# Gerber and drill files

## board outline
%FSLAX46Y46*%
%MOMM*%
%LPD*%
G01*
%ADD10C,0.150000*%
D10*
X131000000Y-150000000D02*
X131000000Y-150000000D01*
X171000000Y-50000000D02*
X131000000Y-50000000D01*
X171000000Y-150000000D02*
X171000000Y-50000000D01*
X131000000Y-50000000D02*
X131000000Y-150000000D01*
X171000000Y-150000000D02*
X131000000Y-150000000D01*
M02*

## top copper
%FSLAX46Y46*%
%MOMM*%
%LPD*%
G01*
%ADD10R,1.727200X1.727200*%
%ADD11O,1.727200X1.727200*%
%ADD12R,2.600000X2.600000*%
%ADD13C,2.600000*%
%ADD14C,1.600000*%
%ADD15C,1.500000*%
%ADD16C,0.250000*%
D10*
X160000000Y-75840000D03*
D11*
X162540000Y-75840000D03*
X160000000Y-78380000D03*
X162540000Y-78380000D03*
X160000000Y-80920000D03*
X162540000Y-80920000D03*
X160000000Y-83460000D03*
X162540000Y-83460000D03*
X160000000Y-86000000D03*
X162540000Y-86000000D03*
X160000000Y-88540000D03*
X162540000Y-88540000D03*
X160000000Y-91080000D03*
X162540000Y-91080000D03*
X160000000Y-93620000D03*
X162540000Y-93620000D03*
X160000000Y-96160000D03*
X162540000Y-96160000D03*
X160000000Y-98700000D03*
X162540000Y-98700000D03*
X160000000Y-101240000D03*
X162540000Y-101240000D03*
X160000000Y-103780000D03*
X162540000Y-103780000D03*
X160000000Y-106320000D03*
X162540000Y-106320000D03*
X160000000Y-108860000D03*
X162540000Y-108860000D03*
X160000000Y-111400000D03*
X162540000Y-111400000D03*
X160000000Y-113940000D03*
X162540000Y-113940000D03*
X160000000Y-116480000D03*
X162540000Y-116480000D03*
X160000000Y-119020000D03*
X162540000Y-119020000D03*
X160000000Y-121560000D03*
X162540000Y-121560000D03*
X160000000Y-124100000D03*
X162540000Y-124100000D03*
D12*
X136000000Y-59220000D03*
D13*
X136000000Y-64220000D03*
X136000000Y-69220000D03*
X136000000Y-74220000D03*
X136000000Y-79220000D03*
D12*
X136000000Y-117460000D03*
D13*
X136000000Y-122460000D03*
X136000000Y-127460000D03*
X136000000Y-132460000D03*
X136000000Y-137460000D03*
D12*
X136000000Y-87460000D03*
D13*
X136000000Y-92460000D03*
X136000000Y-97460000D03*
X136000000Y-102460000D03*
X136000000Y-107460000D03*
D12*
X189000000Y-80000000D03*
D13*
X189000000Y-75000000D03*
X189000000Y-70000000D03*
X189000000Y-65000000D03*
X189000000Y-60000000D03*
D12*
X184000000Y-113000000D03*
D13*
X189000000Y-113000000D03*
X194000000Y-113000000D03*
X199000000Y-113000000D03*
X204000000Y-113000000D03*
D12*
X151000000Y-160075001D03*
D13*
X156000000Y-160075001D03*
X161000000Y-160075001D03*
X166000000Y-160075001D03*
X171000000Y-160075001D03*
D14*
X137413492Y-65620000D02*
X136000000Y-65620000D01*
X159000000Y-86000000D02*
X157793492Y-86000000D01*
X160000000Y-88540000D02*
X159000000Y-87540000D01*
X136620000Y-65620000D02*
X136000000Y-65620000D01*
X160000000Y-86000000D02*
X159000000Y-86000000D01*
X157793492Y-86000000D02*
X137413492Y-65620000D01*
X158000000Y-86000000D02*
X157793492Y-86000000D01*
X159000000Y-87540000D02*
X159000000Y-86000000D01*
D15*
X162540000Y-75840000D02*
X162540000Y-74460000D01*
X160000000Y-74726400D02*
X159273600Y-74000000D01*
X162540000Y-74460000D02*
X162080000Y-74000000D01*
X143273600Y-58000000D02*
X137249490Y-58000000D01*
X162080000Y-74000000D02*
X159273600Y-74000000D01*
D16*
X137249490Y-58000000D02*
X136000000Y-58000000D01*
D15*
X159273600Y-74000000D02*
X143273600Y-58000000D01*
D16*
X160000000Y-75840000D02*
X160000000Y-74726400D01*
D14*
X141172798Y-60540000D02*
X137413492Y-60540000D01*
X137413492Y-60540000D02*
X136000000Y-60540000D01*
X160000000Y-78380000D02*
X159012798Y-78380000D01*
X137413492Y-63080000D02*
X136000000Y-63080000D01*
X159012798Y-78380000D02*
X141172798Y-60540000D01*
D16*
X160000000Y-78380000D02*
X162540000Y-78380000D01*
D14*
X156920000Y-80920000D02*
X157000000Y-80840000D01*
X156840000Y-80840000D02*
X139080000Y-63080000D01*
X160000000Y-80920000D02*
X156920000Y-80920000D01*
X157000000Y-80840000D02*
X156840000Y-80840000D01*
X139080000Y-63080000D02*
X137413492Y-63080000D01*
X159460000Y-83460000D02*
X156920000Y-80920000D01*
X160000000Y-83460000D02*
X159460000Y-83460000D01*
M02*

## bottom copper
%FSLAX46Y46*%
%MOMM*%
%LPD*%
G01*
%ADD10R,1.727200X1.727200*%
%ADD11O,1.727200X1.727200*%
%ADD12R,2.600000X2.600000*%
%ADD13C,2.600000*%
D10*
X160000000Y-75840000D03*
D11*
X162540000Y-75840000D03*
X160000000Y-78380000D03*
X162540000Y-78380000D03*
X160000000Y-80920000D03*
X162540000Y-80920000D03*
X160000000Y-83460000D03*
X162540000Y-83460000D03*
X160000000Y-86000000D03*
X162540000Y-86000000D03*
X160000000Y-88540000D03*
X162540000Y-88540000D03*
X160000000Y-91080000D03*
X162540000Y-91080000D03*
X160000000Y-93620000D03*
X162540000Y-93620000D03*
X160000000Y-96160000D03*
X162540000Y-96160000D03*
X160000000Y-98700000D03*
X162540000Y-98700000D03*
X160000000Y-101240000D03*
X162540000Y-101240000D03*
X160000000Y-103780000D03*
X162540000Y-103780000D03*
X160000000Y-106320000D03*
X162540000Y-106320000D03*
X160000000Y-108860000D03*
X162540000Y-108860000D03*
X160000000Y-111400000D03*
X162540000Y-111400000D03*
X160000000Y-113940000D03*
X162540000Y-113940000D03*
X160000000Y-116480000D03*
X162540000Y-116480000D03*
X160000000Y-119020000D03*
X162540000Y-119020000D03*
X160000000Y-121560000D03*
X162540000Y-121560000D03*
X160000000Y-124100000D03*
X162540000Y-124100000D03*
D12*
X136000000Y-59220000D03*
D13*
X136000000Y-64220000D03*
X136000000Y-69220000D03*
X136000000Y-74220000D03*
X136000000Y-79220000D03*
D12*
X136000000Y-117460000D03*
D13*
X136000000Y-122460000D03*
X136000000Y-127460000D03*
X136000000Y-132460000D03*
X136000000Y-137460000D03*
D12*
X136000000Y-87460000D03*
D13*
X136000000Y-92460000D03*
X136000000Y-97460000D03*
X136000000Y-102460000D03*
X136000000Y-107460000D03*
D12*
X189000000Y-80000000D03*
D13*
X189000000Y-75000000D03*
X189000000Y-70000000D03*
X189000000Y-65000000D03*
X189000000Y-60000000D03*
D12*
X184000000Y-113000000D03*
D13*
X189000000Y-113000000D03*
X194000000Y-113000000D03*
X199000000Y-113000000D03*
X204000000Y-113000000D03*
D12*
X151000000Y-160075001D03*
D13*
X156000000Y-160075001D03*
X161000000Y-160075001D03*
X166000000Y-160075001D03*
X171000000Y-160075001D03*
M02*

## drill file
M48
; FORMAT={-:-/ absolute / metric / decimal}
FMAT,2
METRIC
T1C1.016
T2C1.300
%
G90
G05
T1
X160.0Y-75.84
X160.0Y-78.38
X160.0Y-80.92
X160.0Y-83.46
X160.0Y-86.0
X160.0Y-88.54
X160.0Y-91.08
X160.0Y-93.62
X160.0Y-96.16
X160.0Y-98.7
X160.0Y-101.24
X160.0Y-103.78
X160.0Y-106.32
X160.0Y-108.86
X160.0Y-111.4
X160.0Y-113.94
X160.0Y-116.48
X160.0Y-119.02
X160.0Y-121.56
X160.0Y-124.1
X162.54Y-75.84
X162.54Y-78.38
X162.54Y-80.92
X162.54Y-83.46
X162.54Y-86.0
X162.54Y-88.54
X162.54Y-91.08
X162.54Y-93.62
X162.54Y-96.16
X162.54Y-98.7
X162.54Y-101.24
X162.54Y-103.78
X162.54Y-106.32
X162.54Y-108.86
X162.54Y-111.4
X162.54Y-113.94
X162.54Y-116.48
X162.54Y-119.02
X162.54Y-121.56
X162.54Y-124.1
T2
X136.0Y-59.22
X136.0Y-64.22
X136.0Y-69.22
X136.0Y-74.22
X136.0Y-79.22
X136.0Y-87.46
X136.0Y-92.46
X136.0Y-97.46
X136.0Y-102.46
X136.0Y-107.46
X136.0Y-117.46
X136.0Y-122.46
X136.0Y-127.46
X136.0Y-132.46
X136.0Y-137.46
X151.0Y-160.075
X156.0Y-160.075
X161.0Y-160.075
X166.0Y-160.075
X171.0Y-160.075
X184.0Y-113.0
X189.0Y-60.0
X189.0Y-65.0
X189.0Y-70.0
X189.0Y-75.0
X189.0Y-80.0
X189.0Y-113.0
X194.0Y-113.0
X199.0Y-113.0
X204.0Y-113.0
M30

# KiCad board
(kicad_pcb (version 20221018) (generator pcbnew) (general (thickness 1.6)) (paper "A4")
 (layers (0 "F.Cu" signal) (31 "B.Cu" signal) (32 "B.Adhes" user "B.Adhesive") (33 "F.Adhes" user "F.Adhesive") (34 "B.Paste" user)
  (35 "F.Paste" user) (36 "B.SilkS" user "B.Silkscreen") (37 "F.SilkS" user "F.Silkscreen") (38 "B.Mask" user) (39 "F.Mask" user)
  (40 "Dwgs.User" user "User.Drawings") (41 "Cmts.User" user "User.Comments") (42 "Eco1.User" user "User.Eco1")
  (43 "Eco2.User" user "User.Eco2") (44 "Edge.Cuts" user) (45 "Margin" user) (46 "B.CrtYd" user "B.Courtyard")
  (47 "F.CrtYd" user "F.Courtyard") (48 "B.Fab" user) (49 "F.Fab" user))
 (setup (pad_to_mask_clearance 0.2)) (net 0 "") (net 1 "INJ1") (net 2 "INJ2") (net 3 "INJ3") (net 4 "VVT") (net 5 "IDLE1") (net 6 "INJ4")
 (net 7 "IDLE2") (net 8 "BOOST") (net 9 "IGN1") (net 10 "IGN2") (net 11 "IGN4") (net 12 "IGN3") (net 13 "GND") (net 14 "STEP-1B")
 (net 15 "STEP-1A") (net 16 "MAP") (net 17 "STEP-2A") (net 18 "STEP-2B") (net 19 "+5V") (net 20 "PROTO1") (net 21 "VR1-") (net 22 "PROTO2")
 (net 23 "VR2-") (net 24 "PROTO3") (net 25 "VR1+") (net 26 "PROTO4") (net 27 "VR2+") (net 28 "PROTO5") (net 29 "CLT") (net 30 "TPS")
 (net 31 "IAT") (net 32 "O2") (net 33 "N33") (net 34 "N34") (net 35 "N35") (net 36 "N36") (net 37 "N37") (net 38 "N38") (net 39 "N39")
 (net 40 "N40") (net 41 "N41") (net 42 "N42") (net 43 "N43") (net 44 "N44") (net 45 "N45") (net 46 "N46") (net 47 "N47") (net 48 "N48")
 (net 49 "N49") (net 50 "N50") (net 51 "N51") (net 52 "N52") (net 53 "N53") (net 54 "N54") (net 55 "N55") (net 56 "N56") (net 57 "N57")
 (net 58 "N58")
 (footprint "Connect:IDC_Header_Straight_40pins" (layer "F.Cu") (at 160 75.84 -90)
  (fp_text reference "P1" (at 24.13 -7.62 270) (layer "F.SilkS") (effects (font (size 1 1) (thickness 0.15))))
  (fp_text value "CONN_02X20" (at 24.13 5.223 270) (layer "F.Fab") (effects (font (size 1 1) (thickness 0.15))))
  (pad "1" thru_hole rect (at 0 0 270) (size 1.7272 1.7272) (drill 1.016) (layers "*.Cu" "*.Mask") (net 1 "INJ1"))
  (pad "2" thru_hole oval (at 0 -2.54 270) (size 1.7272 1.7272) (drill 1.016) (layers "*.Cu" "*.Mask") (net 1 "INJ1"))
  (pad "3" thru_hole oval (at 2.54 0 270) (size 1.7272 1.7272) (drill 1.016) (layers "*.Cu" "*.Mask") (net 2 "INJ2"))
  (pad "4" thru_hole oval (at 2.54 -2.54 270) (size 1.7272 1.7272) (drill 1.016) (layers "*.Cu" "*.Mask") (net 2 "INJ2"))
  (pad "5" thru_hole oval (at 5.08 0 270) (size 1.7272 1.7272) (drill 1.016) (layers "*.Cu" "*.Mask") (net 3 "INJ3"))
  (pad "6" thru_hole oval (at 5.08 -2.54 270) (size 1.7272 1.7272) (drill 1.016) (layers "*.Cu" "*.Mask") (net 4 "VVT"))
  (pad "7" thru_hole oval (at 7.62 0 270) (size 1.7272 1.7272) (drill 1.016) (layers "*.Cu" "*.Mask") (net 3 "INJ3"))
  (pad "8" thru_hole oval (at 7.62 -2.54 270) (size 1.7272 1.7272) (drill 1.016) (layers "*.Cu" "*.Mask") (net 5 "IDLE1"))
  (pad "9" thru_hole oval (at 10.16 0 270) (size 1.7272 1.7272) (drill 1.016) (layers "*.Cu" "*.Mask") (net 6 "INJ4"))
  (pad "10" thru_hole oval (at 10.16 -2.54 270) (size 1.7272 1.7272) (drill 1.016) (layers "*.Cu" "*.Mask") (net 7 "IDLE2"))
  (pad "11" thru_hole oval (at 12.7 0 270) (size 1.7272 1.7272) (drill 1.016) (layers "*.Cu" "*.Mask") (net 6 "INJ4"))
  (pad "12" thru_hole oval (at 12.7 -2.54 270) (size 1.7272 1.7272) (drill 1.016) (layers "*.Cu" "*.Mask") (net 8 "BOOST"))
  (pad "13" thru_hole oval (at 15.24 0 270) (size 1.7272 1.7272) (drill 1.016) (layers "*.Cu" "*.Mask") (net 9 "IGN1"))
  (pad "14" thru_hole oval (at 15.24 -2.54 270) (size 1.7272 1.7272) (drill 1.016) (layers "*.Cu" "*.Mask") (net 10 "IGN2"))
  (pad "15" thru_hole oval (at 17.78 0 270) (size 1.7272 1.7272) (drill 1.016) (layers "*.Cu" "*.Mask") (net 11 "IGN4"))
  (pad "16" thru_hole oval (at 17.78 -2.54 270) (size 1.7272 1.7272) (drill 1.016) (layers "*.Cu" "*.Mask") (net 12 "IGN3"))
  (pad "17" thru_hole oval (at 20.32 0 270) (size 1.7272 1.7272) (drill 1.016) (layers "*.Cu" "*.Mask") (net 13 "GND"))
  (pad "18" thru_hole oval (at 20.32 -2.54 270) (size 1.7272 1.7272) (drill 1.016) (layers "*.Cu" "*.Mask") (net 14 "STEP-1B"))
  (pad "19" thru_hole oval (at 22.86 0 270) (size 1.7272 1.7272) (drill 1.016) (layers "*.Cu" "*.Mask") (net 13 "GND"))
  (pad "20" thru_hole oval (at 22.86 -2.54 270) (size 1.7272 1.7272) (drill 1.016) (layers "*.Cu" "*.Mask") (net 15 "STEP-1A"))
  (pad "21" thru_hole oval (at 25.4 0 270) (size 1.7272 1.7272) (drill 1.016) (layers "*.Cu" "*.Mask") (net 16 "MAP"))
  (pad "22" thru_hole oval (at 25.4 -2.54 270) (size 1.7272 1.7272) (drill 1.016) (layers "*.Cu" "*.Mask") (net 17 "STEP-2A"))
  (pad "23" thru_hole oval (at 27.94 0 270) (size 1.7272 1.7272) (drill 1.016) (layers "*.Cu" "*.Mask") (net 13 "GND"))
  (pad "24" thru_hole oval (at 27.94 -2.54 270) (size 1.7272 1.7272) (drill 1.016) (layers "*.Cu" "*.Mask") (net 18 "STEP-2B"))
  (pad "25" thru_hole oval (at 30.48 0 270) (size 1.7272 1.7272) (drill 1.016) (layers "*.Cu" "*.Mask") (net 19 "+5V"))
  (pad "26" thru_hole oval (at 30.48 -2.54 270) (size 1.7272 1.7272) (drill 1.016) (layers "*.Cu" "*.Mask") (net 19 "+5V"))
  (pad "27" thru_hole oval (at 33.02 0 270) (size 1.7272 1.7272) (drill 1.016) (layers "*.Cu" "*.Mask") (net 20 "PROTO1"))
  (pad "28" thru_hole oval (at 33.02 -2.54 270) (size 1.7272 1.7272) (drill 1.016) (layers "*.Cu" "*.Mask") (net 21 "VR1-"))
  (pad "29" thru_hole oval (at 35.56 0 270) (size 1.7272 1.7272) (drill 1.016) (layers "*.Cu" "*.Mask") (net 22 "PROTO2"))
  (pad "30" thru_hole oval (at 35.56 -2.54 270) (size 1.7272 1.7272) (drill 1.016) (layers "*.Cu" "*.Mask") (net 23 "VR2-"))
  (pad "31" thru_hole oval (at 38.1 0 270) (size 1.7272 1.7272) (drill 1.016) (layers "*.Cu" "*.Mask") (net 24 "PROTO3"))
  (pad "32" thru_hole oval (at 38.1 -2.54 270) (size 1.7272 1.7272) (drill 1.016) (layers "*.Cu" "*.Mask") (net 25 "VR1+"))
  (pad "33" thru_hole oval (at 40.64 0 270) (size 1.7272 1.7272) (drill 1.016) (layers "*.Cu" "*.Mask") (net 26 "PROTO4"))
  (pad "34" thru_hole oval (at 40.64 -2.54 270) (size 1.7272 1.7272) (drill 1.016) (layers "*.Cu" "*.Mask") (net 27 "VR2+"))
  (pad "35" thru_hole oval (at 43.18 0 270) (size 1.7272 1.7272) (drill 1.016) (layers "*.Cu" "*.Mask") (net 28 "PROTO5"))
  (pad "36" thru_hole oval (at 43.18 -2.54 270) (size 1.7272 1.7272) (drill 1.016) (layers "*.Cu" "*.Mask") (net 13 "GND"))
  (pad "37" thru_hole oval (at 45.72 0 270) (size 1.7272 1.7272) (drill 1.016) (layers "*.Cu" "*.Mask") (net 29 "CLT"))
  (pad "38" thru_hole oval (at 45.72 -2.54 270) (size 1.7272 1.7272) (drill 1.016) (layers "*.Cu" "*.Mask") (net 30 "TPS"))
  (pad "39" thru_hole oval (at 48.26 0 270) (size 1.7272 1.7272) (drill 1.016) (layers "*.Cu" "*.Mask") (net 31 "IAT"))
  (pad "40" thru_hole oval (at 48.26 -2.54 270) (size 1.7272 1.7272) (drill 1.016) (layers "*.Cu" "*.Mask") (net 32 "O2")))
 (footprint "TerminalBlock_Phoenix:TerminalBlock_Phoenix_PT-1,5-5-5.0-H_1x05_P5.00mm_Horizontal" (layer "F.Cu") (at 136 59.22 -90)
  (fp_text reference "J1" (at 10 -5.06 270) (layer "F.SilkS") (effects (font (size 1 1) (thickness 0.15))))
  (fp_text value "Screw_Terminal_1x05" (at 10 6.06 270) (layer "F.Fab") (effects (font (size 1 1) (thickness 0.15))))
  (pad "1" thru_hole rect (at 0 0 270) (size 2.6 2.6) (drill 1.3) (layers "*.Cu" "*.Mask") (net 1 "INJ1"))
  (pad "2" thru_hole circle (at 5 0 270) (size 2.6 2.6) (drill 1.3) (layers "*.Cu" "*.Mask") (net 2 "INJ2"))
  (pad "3" thru_hole circle (at 10 0 270) (size 2.6 2.6) (drill 1.3) (layers "*.Cu" "*.Mask") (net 3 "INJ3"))
  (pad "4" thru_hole circle (at 15 0 270) (size 2.6 2.6) (drill 1.3) (layers "*.Cu" "*.Mask") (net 6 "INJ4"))
  (pad "5" thru_hole circle (at 20 0 270) (size 2.6 2.6) (drill 1.3) (layers "*.Cu" "*.Mask") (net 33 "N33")))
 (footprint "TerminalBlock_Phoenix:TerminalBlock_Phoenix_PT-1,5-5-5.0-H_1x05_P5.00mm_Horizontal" (layer "F.Cu") (at 136 117.46 -90)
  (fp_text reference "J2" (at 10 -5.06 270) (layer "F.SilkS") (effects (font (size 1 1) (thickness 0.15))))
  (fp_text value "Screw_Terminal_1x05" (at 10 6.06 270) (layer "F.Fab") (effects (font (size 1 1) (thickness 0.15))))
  (pad "1" thru_hole rect (at 0 0 270) (size 2.6 2.6) (drill 1.3) (layers "*.Cu" "*.Mask") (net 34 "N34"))
  (pad "2" thru_hole circle (at 5 0 270) (size 2.6 2.6) (drill 1.3) (layers "*.Cu" "*.Mask") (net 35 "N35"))
  (pad "3" thru_hole circle (at 10 0 270) (size 2.6 2.6) (drill 1.3) (layers "*.Cu" "*.Mask") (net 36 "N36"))
  (pad "4" thru_hole circle (at 15 0 270) (size 2.6 2.6) (drill 1.3) (layers "*.Cu" "*.Mask") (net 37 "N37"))
  (pad "5" thru_hole circle (at 20 0 270) (size 2.6 2.6) (drill 1.3) (layers "*.Cu" "*.Mask") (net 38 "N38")))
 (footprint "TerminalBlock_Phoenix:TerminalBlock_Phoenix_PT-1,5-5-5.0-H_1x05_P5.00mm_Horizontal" (layer "F.Cu") (at 136 87.46 -90)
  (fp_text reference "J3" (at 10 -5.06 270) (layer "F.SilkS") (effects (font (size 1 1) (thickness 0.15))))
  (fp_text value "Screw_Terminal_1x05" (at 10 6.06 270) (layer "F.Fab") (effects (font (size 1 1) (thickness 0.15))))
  (pad "1" thru_hole rect (at 0 0 270) (size 2.6 2.6) (drill 1.3) (layers "*.Cu" "*.Mask") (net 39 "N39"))
  (pad "2" thru_hole circle (at 5 0 270) (size 2.6 2.6) (drill 1.3) (layers "*.Cu" "*.Mask") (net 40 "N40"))
  (pad "3" thru_hole circle (at 10 0 270) (size 2.6 2.6) (drill 1.3) (layers "*.Cu" "*.Mask") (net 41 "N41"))
  (pad "4" thru_hole circle (at 15 0 270) (size 2.6 2.6) (drill 1.3) (layers "*.Cu" "*.Mask") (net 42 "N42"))
  (pad "5" thru_hole circle (at 20 0 270) (size 2.6 2.6) (drill 1.3) (layers "*.Cu" "*.Mask") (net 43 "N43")))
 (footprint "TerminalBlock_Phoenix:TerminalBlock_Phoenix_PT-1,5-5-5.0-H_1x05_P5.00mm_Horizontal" (layer "F.Cu") (at 189 80 90)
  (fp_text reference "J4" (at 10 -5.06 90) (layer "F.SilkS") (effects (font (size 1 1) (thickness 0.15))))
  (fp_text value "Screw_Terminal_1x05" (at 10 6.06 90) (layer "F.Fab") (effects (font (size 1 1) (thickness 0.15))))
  (pad "1" thru_hole rect (at 0 0 90) (size 2.6 2.6) (drill 1.3) (layers "*.Cu" "*.Mask") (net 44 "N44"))
  (pad "2" thru_hole circle (at 5 0 90) (size 2.6 2.6) (drill 1.3) (layers "*.Cu" "*.Mask") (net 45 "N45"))
  (pad "3" thru_hole circle (at 10 0 90) (size 2.6 2.6) (drill 1.3) (layers "*.Cu" "*.Mask") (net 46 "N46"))
  (pad "4" thru_hole circle (at 15 0 90) (size 2.6 2.6) (drill 1.3) (layers "*.Cu" "*.Mask") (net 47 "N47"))
  (pad "5" thru_hole circle (at 20 0 90) (size 2.6 2.6) (drill 1.3) (layers "*.Cu" "*.Mask") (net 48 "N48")))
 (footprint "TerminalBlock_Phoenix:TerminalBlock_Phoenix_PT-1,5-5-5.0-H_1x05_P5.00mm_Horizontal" (layer "F.Cu") (at 184 113)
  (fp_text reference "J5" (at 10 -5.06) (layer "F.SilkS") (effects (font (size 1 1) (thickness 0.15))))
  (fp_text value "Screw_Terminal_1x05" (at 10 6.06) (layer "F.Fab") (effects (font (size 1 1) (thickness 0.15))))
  (pad "1" thru_hole rect (at 0 0) (size 2.6 2.6) (drill 1.3) (layers "*.Cu" "*.Mask") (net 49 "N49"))
  (pad "2" thru_hole circle (at 5 0) (size 2.6 2.6) (drill 1.3) (layers "*.Cu" "*.Mask") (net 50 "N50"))
  (pad "3" thru_hole circle (at 10 0) (size 2.6 2.6) (drill 1.3) (layers "*.Cu" "*.Mask") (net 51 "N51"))
  (pad "4" thru_hole circle (at 15 0) (size 2.6 2.6) (drill 1.3) (layers "*.Cu" "*.Mask") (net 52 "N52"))
  (pad "5" thru_hole circle (at 20 0) (size 2.6 2.6) (drill 1.3) (layers "*.Cu" "*.Mask") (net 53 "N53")))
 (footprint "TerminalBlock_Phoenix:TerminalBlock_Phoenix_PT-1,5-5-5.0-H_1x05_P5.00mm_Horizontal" (layer "F.Cu") (at 151 160.075001)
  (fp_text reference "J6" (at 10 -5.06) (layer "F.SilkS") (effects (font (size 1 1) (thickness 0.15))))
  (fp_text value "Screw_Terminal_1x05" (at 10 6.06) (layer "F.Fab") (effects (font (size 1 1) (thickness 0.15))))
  (pad "1" thru_hole rect (at 0 0) (size 2.6 2.6) (drill 1.3) (layers "*.Cu" "*.Mask") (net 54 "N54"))
  (pad "2" thru_hole circle (at 5 0) (size 2.6 2.6) (drill 1.3) (layers "*.Cu" "*.Mask") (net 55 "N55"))
  (pad "3" thru_hole circle (at 10 0) (size 2.6 2.6) (drill 1.3) (layers "*.Cu" "*.Mask") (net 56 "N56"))
  (pad "4" thru_hole circle (at 15 0) (size 2.6 2.6) (drill 1.3) (layers "*.Cu" "*.Mask") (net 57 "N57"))
  (pad "5" thru_hole circle (at 20 0) (size 2.6 2.6) (drill 1.3) (layers "*.Cu" "*.Mask") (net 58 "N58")))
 (gr_line (start 131 150) (end 131 150) (stroke (width 0.15) (type solid)) (layer "Edge.Cuts"))
 (gr_line (start 171 50) (end 131 50) (stroke (width 0.15) (type solid)) (layer "Edge.Cuts"))
 (gr_line (start 171 150) (end 171 50) (stroke (width 0.15) (type solid)) (layer "Edge.Cuts"))
 (gr_line (start 131 50) (end 131 150) (stroke (width 0.15) (type solid)) (layer "Edge.Cuts"))
 (gr_line (start 171 150) (end 131 150) (stroke (width 0.15) (type solid)) (layer "Edge.Cuts"))
 (segment (start 137.413492 65.62) (end 136 65.62) (width 1.6) (layer "F.Cu") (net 6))
 (segment (start 159 86) (end 157.793492 86) (width 1.6) (layer "F.Cu") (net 6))
 (segment (start 160 88.54) (end 159 87.54) (width 1.6) (layer "F.Cu") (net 6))
 (segment (start 136.62 65.62) (end 136 65.62) (width 1.6) (layer "F.Cu") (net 6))
 (segment (start 160 86) (end 159 86) (width 1.6) (layer "F.Cu") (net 6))
 (segment (start 157.793492 86) (end 137.413492 65.62) (width 1.6) (layer "F.Cu") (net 6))
 (segment (start 158 86) (end 157.793492 86) (width 1.6) (layer "F.Cu") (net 6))
 (segment (start 159 87.54) (end 159 86) (width 1.6) (layer "F.Cu") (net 6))
 (segment (start 162.54 75.84) (end 162.54 74.46) (width 1.5) (layer "F.Cu") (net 1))
 (segment (start 160 74.7264) (end 159.2736 74) (width 1.5) (layer "F.Cu") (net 1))
 (segment (start 162.54 74.46) (end 162.08 74) (width 1.5) (layer "F.Cu") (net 1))
 (segment (start 143.2736 58) (end 137.24949 58) (width 1.5) (layer "F.Cu") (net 1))
 (segment (start 162.08 74) (end 159.2736 74) (width 1.5) (layer "F.Cu") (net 1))
 (segment (start 137.24949 58) (end 136 58) (width 0.25) (layer "F.Cu") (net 1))
 (segment (start 159.2736 74) (end 143.2736 58) (width 1.5) (layer "F.Cu") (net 1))
 (segment (start 160 75.84) (end 160 74.7264) (width 0.25) (layer "F.Cu") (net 1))
 (segment (start 141.172798 60.54) (end 137.413492 60.54) (width 1.6) (layer "F.Cu") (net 2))
 (segment (start 137.413492 60.54) (end 136 60.54) (width 1.6) (layer "F.Cu") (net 2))
 (segment (start 160 78.38) (end 159.012798 78.38) (width 1.6) (layer "F.Cu") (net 2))
 (segment (start 137.413492 63.08) (end 136 63.08) (width 1.6) (layer "F.Cu") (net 2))
 (segment (start 159.012798 78.38) (end 141.172798 60.54) (width 1.6) (layer "F.Cu") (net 2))
 (segment (start 160 78.38) (end 162.54 78.38) (width 0.25) (layer "F.Cu") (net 2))
 (segment (start 156.92 80.92) (end 157 80.84) (width 1.6) (layer "F.Cu") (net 3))
 (segment (start 156.84 80.84) (end 139.08 63.08) (width 1.6) (layer "F.Cu") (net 3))
 (segment (start 160 80.92) (end 156.92 80.92) (width 1.6) (layer "F.Cu") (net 3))
 (segment (start 157 80.84) (end 156.84 80.84) (width 1.6) (layer "F.Cu") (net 3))
 (segment (start 139.08 63.08) (end 137.413492 63.08) (width 1.6) (layer "F.Cu") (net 3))
 (segment (start 159.46 83.46) (end 156.92 80.92) (width 1.6) (layer "F.Cu") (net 3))
 (segment (start 160 83.46) (end 159.46 83.46) (width 1.6) (layer "F.Cu") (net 3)))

